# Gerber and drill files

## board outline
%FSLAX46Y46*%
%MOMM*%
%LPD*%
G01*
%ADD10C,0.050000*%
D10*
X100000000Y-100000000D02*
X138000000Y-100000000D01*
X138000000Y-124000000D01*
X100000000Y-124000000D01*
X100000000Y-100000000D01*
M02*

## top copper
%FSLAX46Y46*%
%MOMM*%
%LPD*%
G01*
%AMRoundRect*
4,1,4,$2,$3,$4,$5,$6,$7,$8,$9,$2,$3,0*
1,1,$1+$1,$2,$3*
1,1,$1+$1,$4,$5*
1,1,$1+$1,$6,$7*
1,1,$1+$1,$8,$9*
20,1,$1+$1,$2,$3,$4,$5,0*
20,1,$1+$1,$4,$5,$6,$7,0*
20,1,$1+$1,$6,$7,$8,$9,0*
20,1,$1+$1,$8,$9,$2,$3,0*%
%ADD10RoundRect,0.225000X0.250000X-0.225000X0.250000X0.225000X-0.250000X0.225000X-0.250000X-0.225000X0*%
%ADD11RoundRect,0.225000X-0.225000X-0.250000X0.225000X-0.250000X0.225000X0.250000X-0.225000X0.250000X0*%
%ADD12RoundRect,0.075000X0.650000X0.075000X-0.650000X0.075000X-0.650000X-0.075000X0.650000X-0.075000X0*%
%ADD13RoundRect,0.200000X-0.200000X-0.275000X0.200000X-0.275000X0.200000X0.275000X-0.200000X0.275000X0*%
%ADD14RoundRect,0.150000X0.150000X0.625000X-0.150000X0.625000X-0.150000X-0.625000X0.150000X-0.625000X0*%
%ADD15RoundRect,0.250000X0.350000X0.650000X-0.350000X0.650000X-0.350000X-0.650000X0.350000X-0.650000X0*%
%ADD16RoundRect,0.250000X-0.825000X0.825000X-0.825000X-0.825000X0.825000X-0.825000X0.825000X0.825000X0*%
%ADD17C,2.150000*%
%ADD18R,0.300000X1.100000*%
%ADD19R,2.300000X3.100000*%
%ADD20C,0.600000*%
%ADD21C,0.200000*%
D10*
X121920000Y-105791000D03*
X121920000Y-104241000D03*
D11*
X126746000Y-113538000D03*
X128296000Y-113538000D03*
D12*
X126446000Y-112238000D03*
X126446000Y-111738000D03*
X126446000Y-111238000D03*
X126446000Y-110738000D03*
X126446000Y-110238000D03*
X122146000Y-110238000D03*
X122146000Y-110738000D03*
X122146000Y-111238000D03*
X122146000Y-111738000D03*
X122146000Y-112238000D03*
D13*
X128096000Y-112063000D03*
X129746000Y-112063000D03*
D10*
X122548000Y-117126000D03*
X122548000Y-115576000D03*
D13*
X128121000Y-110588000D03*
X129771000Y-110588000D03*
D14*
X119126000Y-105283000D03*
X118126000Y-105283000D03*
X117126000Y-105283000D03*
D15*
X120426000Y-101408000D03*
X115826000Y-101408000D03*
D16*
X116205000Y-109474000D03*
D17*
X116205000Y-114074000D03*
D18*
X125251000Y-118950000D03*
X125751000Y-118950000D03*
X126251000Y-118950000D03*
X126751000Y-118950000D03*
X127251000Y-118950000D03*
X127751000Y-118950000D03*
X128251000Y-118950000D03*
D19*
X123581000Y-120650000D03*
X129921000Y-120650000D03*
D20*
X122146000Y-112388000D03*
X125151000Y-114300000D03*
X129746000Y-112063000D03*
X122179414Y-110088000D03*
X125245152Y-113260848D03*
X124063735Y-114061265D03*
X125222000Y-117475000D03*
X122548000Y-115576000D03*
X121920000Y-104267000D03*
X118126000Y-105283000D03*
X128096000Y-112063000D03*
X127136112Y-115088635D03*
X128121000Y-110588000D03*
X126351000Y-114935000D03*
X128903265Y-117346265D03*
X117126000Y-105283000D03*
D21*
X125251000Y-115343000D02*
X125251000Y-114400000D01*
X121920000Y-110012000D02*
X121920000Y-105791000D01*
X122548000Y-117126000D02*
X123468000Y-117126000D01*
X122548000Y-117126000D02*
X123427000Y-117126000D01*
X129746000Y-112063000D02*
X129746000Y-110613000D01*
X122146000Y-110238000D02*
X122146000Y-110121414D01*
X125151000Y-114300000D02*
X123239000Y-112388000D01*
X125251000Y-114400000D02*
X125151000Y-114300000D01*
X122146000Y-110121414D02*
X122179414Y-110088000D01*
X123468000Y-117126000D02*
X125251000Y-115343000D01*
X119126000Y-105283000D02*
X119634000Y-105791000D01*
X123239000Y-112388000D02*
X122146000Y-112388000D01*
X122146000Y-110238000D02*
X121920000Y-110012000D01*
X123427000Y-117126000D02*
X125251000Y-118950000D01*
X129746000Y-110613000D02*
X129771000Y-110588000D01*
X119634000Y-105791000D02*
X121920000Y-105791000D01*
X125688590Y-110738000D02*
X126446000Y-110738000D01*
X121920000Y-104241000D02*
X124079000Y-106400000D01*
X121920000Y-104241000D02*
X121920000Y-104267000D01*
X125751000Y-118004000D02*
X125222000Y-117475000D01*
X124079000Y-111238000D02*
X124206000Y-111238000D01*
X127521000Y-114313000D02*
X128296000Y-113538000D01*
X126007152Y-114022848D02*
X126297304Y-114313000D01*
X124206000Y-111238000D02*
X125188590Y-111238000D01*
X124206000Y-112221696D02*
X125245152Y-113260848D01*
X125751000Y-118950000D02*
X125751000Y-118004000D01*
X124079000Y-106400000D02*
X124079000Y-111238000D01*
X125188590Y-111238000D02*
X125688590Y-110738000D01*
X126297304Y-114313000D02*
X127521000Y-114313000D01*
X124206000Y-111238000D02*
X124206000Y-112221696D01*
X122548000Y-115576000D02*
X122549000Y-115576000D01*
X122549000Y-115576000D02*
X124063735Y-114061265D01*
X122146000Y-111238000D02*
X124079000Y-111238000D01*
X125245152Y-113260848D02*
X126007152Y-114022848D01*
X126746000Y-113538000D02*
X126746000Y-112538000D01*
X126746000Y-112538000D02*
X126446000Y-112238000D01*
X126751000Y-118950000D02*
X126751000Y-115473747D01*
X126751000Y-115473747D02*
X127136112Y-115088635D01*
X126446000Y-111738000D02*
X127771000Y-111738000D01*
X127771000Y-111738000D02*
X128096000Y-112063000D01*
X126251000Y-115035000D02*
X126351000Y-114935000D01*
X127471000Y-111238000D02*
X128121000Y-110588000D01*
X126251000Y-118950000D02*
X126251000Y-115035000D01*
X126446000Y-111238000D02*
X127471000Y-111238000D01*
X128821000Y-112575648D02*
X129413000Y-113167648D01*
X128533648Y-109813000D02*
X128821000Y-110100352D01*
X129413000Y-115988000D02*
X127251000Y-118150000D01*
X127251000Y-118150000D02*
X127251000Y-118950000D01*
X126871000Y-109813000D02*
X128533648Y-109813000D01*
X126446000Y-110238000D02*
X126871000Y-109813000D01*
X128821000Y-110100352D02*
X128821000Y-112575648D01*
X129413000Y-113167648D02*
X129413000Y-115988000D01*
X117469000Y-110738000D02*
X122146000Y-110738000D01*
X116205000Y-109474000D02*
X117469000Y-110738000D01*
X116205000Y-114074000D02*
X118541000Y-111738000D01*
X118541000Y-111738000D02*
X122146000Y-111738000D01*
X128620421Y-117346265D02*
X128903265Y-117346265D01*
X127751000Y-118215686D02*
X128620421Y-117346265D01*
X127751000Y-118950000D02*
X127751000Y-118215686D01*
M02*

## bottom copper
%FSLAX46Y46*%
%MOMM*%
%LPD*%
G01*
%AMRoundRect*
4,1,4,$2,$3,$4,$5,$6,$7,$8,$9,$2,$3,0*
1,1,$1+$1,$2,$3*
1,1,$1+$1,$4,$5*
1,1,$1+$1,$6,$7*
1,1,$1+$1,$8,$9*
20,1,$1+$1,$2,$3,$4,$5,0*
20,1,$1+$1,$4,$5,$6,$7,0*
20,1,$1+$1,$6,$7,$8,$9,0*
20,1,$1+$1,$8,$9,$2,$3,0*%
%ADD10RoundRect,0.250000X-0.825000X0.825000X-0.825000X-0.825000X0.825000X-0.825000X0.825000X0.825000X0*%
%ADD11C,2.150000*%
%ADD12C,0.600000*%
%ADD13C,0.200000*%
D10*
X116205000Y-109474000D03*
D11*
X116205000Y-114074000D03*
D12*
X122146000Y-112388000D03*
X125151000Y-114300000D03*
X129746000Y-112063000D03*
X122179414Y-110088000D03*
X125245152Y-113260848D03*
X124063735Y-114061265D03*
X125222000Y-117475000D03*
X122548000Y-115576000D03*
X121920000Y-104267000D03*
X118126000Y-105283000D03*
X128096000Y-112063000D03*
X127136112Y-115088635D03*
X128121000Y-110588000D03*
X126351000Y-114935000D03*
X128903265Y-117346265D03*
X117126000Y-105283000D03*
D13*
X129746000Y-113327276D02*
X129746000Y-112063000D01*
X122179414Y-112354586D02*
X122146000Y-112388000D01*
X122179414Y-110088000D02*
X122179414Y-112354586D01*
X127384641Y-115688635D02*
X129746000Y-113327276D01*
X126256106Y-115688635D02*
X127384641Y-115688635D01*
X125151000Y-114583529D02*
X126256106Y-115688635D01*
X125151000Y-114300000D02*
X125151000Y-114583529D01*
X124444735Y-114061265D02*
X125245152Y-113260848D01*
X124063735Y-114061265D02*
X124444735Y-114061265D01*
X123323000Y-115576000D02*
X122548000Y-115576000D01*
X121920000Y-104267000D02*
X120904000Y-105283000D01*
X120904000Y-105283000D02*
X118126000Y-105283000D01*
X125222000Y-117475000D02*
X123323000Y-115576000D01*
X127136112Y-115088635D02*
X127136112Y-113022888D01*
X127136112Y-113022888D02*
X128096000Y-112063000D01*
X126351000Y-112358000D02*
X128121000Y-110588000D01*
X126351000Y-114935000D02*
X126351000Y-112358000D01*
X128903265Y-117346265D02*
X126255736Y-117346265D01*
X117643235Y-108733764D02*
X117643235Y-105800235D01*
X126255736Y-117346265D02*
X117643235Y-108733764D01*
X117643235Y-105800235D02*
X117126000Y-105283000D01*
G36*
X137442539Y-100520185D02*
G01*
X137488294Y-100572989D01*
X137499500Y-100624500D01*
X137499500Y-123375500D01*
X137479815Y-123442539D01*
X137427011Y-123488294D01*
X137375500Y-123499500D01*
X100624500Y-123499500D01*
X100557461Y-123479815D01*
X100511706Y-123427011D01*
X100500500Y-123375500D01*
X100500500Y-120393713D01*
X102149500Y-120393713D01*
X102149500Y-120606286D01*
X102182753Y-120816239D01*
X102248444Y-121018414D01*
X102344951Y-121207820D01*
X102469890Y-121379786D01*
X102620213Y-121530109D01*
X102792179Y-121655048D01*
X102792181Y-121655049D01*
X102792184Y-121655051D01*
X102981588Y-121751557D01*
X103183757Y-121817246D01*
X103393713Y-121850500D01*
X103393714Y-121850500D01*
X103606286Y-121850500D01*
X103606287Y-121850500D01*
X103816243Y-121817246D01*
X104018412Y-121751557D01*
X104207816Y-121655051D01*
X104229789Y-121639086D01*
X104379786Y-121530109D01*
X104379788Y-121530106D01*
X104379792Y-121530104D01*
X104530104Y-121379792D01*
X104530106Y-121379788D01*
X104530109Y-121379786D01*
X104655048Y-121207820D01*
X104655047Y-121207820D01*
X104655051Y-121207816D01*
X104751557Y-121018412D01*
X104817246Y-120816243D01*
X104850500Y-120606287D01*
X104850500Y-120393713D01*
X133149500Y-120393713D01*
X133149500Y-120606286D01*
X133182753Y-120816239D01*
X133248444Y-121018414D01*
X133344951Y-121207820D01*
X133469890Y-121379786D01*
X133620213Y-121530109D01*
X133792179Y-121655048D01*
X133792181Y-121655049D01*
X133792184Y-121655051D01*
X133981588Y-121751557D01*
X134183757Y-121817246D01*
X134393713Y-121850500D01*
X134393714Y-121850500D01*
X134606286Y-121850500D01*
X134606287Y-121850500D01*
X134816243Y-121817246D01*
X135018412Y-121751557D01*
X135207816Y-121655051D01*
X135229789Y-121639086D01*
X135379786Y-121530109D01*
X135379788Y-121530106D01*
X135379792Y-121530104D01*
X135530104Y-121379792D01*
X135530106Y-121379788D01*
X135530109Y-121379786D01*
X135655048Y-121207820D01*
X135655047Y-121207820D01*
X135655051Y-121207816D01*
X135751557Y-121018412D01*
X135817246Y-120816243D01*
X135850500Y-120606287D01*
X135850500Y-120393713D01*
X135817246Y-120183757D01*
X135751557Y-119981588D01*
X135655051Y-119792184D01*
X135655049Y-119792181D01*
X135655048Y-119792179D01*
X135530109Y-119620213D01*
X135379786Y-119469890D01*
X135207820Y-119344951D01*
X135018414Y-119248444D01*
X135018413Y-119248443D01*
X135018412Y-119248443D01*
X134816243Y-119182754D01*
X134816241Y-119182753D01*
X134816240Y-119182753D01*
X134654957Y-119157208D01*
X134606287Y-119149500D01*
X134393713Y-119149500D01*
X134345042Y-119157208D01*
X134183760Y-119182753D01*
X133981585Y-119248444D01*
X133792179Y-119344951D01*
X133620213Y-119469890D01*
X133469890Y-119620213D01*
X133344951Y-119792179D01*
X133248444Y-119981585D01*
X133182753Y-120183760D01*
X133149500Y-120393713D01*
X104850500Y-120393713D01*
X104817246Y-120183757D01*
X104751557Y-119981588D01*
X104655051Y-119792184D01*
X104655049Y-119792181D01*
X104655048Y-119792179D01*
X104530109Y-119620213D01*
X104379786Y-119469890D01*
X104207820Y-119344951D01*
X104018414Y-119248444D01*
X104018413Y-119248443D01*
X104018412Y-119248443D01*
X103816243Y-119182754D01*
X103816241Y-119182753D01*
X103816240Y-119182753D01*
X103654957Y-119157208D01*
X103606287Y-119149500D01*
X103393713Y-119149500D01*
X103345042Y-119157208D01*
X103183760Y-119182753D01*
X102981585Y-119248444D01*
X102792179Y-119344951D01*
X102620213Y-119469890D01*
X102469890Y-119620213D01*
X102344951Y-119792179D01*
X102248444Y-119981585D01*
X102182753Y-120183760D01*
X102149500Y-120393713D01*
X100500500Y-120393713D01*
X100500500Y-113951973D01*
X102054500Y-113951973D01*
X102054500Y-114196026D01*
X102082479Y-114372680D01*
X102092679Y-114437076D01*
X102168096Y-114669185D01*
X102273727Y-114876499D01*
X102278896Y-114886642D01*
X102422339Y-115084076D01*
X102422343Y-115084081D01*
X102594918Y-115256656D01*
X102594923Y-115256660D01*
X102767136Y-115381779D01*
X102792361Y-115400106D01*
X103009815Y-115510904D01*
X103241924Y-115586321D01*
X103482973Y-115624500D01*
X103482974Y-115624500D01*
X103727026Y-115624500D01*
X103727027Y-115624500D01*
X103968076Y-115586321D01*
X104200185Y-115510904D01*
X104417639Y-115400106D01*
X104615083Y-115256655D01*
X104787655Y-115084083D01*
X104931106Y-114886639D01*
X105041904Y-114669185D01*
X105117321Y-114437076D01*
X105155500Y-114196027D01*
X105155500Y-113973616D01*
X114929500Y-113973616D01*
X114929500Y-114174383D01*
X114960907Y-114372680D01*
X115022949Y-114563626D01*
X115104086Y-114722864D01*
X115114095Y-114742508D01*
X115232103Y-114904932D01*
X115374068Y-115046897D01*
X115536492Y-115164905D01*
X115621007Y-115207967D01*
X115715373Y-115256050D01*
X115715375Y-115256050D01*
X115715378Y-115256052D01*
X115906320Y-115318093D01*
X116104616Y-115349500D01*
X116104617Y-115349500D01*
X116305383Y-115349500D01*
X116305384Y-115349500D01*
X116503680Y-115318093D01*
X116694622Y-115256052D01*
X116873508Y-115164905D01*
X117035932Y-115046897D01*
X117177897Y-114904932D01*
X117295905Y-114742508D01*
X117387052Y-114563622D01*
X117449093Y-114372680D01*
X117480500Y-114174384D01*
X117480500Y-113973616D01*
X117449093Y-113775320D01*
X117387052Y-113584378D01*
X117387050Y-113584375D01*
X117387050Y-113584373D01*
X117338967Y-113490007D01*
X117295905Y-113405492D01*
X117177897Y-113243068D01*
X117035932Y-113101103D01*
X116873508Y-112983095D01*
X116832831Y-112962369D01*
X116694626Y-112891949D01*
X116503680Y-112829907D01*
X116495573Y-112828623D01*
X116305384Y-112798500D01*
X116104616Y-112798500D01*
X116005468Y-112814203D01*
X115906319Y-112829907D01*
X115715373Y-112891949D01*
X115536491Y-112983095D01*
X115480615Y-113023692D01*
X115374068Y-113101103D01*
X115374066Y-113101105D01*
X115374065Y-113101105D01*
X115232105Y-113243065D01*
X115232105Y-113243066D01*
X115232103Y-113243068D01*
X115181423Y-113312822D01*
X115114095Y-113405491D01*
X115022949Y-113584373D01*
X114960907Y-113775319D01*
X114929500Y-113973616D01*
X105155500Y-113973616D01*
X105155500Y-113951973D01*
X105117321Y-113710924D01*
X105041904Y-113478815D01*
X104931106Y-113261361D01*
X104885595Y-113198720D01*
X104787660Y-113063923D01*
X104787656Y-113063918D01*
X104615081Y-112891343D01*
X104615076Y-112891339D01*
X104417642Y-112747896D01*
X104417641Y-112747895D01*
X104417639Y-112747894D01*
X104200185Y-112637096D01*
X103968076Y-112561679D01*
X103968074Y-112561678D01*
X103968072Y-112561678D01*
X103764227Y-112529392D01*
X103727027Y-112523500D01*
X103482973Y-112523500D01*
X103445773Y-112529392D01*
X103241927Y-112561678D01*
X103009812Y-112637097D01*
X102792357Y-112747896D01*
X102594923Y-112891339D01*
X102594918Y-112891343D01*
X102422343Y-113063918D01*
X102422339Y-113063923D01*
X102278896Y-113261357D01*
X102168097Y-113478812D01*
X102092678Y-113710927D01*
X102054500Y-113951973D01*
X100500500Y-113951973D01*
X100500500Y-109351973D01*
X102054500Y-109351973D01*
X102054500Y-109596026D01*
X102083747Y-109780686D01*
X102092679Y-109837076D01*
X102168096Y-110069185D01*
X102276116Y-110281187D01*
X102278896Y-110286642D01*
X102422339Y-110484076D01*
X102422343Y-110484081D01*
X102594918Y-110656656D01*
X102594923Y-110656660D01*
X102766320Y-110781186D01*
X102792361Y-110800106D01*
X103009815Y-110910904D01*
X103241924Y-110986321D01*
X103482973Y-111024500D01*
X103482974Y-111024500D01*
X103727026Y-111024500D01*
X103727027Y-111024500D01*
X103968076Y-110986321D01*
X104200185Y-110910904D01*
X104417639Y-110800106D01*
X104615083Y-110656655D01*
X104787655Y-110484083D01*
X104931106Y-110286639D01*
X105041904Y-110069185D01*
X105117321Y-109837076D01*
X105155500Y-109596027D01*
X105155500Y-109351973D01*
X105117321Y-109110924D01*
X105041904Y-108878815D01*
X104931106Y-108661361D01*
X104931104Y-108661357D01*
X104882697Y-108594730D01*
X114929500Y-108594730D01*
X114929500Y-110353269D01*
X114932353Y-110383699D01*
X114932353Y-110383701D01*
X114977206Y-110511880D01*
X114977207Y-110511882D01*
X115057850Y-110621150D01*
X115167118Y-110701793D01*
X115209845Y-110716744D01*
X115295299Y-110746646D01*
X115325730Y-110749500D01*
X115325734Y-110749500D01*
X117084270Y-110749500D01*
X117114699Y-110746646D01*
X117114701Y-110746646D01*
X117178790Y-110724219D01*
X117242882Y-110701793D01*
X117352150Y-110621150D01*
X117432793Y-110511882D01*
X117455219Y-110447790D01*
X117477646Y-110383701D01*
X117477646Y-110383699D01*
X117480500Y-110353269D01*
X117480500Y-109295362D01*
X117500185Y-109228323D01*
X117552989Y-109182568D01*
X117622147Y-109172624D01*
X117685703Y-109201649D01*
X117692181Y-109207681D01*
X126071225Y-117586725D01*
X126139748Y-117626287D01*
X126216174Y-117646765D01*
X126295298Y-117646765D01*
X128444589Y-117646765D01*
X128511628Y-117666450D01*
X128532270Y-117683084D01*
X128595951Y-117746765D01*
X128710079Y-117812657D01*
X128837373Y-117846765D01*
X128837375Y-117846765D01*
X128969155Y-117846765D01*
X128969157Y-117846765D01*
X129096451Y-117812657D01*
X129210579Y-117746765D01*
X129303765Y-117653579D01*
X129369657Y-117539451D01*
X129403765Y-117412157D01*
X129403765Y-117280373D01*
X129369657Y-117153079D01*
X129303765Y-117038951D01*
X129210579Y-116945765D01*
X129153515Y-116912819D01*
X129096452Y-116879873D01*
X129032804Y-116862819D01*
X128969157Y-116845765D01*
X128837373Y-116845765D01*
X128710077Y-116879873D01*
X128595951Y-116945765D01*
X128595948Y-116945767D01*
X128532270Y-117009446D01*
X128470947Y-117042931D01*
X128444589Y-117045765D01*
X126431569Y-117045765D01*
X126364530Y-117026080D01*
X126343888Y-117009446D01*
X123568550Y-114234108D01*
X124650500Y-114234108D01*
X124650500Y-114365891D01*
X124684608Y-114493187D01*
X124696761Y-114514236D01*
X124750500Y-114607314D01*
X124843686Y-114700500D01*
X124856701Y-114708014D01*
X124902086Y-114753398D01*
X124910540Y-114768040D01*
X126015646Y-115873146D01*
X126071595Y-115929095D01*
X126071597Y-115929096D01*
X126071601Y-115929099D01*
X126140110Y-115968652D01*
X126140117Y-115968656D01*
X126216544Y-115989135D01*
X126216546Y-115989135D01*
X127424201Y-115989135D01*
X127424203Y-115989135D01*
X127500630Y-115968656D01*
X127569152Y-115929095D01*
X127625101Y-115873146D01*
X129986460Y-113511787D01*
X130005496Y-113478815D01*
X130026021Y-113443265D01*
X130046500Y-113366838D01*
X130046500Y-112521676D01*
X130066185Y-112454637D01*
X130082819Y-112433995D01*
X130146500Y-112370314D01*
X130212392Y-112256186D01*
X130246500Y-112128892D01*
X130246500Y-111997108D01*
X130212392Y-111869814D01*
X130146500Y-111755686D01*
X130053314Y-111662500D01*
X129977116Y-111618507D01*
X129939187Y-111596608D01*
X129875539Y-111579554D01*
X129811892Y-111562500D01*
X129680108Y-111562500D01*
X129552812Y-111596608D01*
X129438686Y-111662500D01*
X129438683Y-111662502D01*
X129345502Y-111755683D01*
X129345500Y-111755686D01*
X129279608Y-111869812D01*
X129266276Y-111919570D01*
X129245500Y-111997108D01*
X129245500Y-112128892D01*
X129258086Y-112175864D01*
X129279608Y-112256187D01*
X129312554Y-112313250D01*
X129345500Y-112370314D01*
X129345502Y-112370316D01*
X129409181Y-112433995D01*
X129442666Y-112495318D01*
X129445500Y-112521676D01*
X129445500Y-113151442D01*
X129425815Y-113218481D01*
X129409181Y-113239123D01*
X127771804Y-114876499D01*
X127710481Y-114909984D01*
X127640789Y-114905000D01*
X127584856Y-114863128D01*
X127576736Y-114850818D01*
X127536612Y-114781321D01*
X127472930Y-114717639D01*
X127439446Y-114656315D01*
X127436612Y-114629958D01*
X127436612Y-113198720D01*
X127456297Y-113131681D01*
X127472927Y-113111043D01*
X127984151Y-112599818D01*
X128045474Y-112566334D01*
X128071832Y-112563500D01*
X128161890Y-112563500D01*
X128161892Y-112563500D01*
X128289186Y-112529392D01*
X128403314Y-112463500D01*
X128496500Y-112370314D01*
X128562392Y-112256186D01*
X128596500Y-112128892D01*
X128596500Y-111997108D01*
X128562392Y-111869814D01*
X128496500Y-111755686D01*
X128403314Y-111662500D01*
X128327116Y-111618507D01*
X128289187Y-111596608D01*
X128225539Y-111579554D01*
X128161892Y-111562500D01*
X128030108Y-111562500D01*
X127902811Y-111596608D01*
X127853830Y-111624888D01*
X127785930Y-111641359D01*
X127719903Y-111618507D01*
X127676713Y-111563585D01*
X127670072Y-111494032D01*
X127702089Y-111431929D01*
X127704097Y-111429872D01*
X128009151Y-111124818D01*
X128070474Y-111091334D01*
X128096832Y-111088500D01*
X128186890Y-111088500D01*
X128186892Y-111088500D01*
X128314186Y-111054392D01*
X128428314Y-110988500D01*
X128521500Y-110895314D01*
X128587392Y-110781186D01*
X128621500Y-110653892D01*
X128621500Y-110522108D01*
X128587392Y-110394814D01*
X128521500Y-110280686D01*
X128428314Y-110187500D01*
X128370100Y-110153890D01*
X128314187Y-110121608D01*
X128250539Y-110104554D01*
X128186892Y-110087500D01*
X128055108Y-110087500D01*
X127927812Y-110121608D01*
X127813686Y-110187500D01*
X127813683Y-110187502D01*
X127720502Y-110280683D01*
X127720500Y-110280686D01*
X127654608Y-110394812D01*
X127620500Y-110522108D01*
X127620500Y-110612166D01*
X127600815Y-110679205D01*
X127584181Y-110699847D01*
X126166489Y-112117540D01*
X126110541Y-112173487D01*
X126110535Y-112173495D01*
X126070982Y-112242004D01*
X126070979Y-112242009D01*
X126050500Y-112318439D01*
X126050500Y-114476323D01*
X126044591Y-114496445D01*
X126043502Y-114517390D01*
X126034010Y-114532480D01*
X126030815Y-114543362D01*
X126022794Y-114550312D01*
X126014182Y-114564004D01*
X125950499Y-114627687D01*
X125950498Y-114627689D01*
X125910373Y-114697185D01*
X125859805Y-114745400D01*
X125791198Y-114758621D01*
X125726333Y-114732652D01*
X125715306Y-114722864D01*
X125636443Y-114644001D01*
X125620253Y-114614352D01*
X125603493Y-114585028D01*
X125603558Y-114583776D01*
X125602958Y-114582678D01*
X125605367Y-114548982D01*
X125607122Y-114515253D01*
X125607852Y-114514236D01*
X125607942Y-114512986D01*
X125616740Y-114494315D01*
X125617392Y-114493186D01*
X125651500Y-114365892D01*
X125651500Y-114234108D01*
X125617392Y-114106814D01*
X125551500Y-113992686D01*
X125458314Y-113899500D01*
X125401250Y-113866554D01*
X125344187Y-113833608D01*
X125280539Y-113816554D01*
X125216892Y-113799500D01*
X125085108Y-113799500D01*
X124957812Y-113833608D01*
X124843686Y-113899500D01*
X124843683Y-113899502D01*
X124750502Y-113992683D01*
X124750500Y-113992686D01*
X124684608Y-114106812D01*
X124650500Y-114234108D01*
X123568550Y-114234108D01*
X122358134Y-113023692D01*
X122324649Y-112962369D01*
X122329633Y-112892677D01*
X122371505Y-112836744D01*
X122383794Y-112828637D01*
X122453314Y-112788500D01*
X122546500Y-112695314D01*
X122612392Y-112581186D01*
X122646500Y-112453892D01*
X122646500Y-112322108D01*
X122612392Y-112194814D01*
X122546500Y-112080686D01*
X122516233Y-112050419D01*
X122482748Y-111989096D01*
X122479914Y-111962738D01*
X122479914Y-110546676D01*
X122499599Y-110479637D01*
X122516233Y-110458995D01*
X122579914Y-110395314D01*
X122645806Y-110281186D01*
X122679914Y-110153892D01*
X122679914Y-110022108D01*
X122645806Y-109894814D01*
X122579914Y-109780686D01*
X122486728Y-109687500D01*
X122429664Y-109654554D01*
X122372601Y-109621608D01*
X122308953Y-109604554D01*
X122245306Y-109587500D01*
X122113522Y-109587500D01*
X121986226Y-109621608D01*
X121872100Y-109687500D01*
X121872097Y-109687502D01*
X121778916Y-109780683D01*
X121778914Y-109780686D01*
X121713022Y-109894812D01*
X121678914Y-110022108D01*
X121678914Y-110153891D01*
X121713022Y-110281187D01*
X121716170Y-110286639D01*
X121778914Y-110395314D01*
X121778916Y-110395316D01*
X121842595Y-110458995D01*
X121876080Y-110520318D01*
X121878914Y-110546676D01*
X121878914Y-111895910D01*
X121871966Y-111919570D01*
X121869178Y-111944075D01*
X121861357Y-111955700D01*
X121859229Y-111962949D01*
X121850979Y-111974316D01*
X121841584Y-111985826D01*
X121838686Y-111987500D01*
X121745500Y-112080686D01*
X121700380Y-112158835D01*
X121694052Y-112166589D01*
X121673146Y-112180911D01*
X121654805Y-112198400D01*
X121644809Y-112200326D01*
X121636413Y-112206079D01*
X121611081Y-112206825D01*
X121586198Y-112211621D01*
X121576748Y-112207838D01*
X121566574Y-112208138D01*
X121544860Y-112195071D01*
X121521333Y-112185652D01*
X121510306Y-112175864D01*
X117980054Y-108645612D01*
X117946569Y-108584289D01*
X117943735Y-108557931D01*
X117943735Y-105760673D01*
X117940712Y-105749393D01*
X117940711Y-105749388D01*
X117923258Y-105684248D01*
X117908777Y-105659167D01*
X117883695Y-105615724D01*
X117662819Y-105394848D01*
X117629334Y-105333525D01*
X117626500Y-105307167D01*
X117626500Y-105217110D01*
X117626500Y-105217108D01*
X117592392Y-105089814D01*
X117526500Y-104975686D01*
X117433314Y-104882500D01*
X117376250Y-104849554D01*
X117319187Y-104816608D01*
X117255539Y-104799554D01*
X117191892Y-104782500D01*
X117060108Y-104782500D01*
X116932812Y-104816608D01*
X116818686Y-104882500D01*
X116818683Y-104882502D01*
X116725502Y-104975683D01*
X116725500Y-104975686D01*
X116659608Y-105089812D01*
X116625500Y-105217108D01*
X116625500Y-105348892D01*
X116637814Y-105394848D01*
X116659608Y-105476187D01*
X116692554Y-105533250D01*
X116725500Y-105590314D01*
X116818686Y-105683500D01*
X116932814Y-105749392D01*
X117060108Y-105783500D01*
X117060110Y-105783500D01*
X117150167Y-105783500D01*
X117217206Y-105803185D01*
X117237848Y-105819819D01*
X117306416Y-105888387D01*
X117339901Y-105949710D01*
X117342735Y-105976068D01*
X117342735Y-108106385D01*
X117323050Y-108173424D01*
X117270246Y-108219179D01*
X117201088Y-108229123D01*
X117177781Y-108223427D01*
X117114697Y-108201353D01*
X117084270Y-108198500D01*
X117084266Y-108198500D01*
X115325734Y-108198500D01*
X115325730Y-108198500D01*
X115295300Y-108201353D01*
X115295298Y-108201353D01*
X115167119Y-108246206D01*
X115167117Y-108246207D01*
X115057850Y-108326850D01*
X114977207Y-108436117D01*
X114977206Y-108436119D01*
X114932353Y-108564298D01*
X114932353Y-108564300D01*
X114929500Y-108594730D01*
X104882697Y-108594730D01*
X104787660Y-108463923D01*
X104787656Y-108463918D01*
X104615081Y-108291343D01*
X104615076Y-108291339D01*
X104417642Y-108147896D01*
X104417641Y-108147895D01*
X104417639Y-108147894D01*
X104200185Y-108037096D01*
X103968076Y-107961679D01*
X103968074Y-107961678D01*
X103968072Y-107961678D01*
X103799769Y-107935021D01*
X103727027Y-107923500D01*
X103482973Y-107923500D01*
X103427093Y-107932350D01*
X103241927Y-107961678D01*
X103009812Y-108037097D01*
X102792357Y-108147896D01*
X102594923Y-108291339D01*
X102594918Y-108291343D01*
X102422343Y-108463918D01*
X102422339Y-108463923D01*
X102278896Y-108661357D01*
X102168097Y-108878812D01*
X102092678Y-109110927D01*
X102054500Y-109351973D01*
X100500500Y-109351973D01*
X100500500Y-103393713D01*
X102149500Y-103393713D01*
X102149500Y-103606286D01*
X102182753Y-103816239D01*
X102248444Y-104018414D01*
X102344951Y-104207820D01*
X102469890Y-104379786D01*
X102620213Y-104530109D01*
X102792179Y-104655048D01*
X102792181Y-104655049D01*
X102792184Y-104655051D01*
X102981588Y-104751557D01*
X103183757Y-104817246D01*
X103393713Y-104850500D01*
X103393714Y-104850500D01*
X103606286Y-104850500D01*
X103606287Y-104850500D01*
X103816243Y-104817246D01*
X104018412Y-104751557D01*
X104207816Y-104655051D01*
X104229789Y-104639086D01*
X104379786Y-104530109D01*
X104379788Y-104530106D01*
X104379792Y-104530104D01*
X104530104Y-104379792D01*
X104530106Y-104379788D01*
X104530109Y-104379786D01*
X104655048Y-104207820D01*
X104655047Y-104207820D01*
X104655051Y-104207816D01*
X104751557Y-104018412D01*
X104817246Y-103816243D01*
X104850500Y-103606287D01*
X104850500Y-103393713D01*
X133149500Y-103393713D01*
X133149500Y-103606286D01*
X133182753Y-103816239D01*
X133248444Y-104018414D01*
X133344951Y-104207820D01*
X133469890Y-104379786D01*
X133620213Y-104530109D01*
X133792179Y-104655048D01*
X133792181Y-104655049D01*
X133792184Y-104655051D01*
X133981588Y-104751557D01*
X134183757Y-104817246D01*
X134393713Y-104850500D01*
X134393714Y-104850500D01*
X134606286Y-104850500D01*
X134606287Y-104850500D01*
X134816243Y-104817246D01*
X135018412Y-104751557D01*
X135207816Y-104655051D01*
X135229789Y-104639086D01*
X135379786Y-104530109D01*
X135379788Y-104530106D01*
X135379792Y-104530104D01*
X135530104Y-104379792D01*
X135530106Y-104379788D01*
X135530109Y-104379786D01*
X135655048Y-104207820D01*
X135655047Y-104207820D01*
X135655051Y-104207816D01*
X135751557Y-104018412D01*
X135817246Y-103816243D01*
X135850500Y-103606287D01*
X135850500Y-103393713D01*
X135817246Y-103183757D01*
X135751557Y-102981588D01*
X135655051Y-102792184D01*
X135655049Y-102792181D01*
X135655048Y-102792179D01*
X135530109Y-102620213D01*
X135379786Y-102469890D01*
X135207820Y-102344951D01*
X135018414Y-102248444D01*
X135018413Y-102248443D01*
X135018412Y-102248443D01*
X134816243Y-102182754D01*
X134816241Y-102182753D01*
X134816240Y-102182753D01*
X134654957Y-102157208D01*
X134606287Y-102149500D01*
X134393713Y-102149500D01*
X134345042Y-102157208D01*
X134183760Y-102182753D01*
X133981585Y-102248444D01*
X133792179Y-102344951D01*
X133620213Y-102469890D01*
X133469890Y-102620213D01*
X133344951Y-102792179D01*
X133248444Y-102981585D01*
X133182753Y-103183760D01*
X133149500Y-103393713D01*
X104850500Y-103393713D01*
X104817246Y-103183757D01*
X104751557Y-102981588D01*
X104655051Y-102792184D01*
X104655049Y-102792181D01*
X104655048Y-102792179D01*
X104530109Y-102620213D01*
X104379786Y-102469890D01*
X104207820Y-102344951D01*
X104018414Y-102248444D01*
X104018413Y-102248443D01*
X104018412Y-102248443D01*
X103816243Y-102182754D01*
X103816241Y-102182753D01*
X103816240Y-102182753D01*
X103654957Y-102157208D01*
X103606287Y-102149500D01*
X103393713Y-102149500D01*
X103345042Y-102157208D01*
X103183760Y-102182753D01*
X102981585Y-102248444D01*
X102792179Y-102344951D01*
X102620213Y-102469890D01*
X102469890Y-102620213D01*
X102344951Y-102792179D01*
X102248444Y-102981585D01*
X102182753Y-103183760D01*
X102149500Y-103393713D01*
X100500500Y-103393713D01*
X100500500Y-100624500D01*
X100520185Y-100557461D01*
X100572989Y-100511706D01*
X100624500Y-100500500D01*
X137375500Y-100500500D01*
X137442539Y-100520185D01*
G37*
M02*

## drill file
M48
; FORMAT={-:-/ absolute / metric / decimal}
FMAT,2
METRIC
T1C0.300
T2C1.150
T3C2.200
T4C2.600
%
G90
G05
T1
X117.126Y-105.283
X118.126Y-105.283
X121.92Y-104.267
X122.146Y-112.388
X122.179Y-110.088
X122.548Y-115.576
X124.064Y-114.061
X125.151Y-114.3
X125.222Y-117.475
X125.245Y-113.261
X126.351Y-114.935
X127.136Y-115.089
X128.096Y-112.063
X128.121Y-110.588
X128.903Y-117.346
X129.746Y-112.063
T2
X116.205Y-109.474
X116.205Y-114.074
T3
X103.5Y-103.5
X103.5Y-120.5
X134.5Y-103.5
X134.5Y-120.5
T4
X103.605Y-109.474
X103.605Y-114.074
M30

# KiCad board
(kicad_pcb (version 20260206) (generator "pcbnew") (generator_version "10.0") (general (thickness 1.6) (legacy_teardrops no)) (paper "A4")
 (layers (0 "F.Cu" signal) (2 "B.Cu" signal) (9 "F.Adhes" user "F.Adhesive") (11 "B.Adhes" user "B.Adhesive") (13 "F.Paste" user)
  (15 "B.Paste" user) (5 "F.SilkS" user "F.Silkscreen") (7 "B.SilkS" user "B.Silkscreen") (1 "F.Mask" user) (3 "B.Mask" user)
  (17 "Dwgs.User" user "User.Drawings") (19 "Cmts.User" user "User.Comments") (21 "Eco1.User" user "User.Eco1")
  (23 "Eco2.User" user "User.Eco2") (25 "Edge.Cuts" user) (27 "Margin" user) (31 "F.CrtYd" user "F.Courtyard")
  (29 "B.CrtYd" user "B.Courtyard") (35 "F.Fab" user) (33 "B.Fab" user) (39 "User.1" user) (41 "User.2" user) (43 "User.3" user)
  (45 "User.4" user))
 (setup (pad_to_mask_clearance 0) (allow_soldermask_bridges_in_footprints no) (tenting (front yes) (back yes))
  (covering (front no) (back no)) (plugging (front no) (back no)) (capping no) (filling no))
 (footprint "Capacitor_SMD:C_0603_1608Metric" (layer "F.Cu") (at 121.92 105.016 90)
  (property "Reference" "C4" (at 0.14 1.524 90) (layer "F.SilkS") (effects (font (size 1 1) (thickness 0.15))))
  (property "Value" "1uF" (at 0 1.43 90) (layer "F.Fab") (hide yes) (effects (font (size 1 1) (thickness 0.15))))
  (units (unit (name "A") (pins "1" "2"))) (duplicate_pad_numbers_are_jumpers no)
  (pad "1" smd roundrect (at -0.775 0 90) (size 0.9 0.95) (layers "F.Cu" "F.Mask" "F.Paste") (roundrect_rratio 0.25) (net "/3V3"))
  (pad "2" smd roundrect (at 0.775 0 90) (size 0.9 0.95) (layers "F.Cu" "F.Mask" "F.Paste") (roundrect_rratio 0.25) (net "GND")))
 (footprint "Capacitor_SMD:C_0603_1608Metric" (layer "F.Cu") (at 127.521 113.538)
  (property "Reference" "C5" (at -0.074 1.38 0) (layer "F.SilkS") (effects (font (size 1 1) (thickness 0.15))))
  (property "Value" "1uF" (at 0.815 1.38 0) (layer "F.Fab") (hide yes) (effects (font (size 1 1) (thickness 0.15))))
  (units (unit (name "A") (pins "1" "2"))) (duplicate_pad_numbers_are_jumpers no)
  (pad "1" smd roundrect (at -0.775 0) (size 0.9 0.95) (layers "F.Cu" "F.Mask" "F.Paste") (roundrect_rratio 0.25) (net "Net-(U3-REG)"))
  (pad "2" smd roundrect (at 0.775 0) (size 0.9 0.95) (layers "F.Cu" "F.Mask" "F.Paste") (roundrect_rratio 0.25) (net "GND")))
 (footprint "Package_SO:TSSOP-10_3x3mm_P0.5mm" (layer "F.Cu") (at 124.296 111.238 180)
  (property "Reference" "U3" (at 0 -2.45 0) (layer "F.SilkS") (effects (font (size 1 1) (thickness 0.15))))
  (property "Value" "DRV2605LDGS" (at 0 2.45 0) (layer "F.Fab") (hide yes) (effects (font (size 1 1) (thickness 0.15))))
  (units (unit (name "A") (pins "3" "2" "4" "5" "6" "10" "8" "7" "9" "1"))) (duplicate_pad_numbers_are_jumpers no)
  (pad "1" smd roundrect (at -2.15 -1 180) (size 1.45 0.3) (layers "F.Cu" "F.Mask" "F.Paste") (roundrect_rratio 0.25) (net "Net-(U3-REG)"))
  (pad "2" smd roundrect (at -2.15 -0.5 180) (size 1.45 0.3) (layers "F.Cu" "F.Mask" "F.Paste") (roundrect_rratio 0.25) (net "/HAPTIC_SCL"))
  (pad "3" smd roundrect (at -2.15 0 180) (size 1.45 0.3) (layers "F.Cu" "F.Mask" "F.Paste") (roundrect_rratio 0.25) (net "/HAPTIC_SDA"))
  (pad "4" smd roundrect (at -2.15 0.5 180) (size 1.45 0.3) (layers "F.Cu" "F.Mask" "F.Paste") (roundrect_rratio 0.25) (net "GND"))
  (pad "5" smd roundrect (at -2.15 1 180) (size 1.45 0.3) (layers "F.Cu" "F.Mask" "F.Paste") (roundrect_rratio 0.25) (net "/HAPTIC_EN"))
  (pad "6" smd roundrect (at 2.15 1 180) (size 1.45 0.3) (layers "F.Cu" "F.Mask" "F.Paste") (roundrect_rratio 0.25) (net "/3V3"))
  (pad "7" smd roundrect (at 2.15 0.5 180) (size 1.45 0.3) (layers "F.Cu" "F.Mask" "F.Paste") (roundrect_rratio 0.25) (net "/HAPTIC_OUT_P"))
  (pad "8" smd roundrect (at 2.15 0 180) (size 1.45 0.3) (layers "F.Cu" "F.Mask" "F.Paste") (roundrect_rratio 0.25) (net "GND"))
  (pad "9" smd roundrect (at 2.15 -0.5 180) (size 1.45 0.3) (layers "F.Cu" "F.Mask" "F.Paste") (roundrect_rratio 0.25) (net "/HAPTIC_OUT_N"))
  (pad "10" smd roundrect (at 2.15 -1 180) (size 1.45 0.3) (layers "F.Cu" "F.Mask" "F.Paste") (roundrect_rratio 0.25) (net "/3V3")))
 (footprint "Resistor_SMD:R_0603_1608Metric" (layer "F.Cu") (at 128.921 112.063)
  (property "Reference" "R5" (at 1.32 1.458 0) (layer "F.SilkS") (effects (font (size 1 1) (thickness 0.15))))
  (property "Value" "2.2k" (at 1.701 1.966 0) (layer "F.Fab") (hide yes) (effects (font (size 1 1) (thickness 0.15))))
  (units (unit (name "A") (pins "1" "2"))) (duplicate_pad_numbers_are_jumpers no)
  (pad "1" smd roundrect (at -0.825 0) (size 0.8 0.95) (layers "F.Cu" "F.Mask" "F.Paste") (roundrect_rratio 0.25) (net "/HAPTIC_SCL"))
  (pad "2" smd roundrect (at 0.825 0) (size 0.8 0.95) (layers "F.Cu" "F.Mask" "F.Paste") (roundrect_rratio 0.25) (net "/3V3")))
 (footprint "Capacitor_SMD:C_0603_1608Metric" (layer "F.Cu") (at 122.548 116.351 90)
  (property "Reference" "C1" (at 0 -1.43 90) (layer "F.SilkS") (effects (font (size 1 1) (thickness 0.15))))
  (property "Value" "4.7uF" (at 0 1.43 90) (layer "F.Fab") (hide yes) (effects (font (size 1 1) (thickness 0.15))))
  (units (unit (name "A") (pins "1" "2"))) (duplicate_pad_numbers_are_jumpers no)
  (pad "1" smd roundrect (at -0.775 0 90) (size 0.9 0.95) (layers "F.Cu" "F.Mask" "F.Paste") (roundrect_rratio 0.25) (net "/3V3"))
  (pad "2" smd roundrect (at 0.775 0 90) (size 0.9 0.95) (layers "F.Cu" "F.Mask" "F.Paste") (roundrect_rratio 0.25) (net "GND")))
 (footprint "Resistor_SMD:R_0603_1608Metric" (layer "F.Cu") (at 128.946 110.588)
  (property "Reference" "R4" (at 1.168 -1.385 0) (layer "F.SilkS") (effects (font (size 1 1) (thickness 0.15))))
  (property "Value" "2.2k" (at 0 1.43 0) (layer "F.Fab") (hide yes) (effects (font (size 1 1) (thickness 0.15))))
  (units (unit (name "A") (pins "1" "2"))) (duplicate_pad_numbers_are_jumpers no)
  (pad "1" smd roundrect (at -0.825 0) (size 0.8 0.95) (layers "F.Cu" "F.Mask" "F.Paste") (roundrect_rratio 0.25) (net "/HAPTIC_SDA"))
  (pad "2" smd roundrect (at 0.825 0) (size 0.8 0.95) (layers "F.Cu" "F.Mask" "F.Paste") (roundrect_rratio 0.25) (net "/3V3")))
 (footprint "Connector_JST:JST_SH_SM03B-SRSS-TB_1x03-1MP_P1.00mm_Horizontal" (layer "F.Cu") (at 118.126 103.283 180)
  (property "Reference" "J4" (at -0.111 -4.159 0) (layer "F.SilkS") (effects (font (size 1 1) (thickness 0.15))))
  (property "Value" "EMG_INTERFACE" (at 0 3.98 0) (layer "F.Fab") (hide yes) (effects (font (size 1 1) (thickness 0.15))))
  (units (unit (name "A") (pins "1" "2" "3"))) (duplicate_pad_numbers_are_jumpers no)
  (pad "1" smd roundrect (at -1 -2 180) (size 0.6 1.55) (layers "F.Cu" "F.Mask" "F.Paste") (roundrect_rratio 0.25) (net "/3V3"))
  (pad "2" smd roundrect (at 0 -2 180) (size 0.6 1.55) (layers "F.Cu" "F.Mask" "F.Paste") (roundrect_rratio 0.25) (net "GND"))
  (pad "3" smd roundrect (at 1 -2 180) (size 0.6 1.55) (layers "F.Cu" "F.Mask" "F.Paste") (roundrect_rratio 0.25) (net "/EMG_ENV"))
  (pad "MP" smd roundrect (at -2.3 1.875 180) (size 1.2 1.8) (layers "F.Cu" "F.Mask" "F.Paste") (roundrect_rratio 0.208333))
  (pad "MP" smd roundrect (at 2.3 1.875 180) (size 1.2 1.8) (layers "F.Cu" "F.Mask" "F.Paste") (roundrect_rratio 0.208333)))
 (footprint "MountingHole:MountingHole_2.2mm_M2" (layer "F.Cu") (at 103.5 103.5)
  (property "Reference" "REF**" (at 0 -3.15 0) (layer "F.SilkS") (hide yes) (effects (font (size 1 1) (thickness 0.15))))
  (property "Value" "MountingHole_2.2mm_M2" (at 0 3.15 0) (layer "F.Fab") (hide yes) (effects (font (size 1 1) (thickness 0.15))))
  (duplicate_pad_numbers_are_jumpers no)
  (pad "" np_thru_hole circle (at 0 0) (size 2.2 2.2) (drill 2.2) (layers "*.Cu" "*.Mask")))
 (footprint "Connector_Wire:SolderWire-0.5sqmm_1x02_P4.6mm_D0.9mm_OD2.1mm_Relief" (layer "F.Cu") (at 116.205 109.474 -90)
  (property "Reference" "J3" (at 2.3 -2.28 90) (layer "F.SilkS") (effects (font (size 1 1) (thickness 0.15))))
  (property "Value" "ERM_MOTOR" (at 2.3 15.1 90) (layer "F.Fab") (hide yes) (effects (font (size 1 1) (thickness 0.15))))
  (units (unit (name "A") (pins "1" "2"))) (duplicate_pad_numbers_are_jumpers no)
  (pad "" np_thru_hole circle (at 0 12.6 270) (size 2.6 2.6) (drill 2.6) (layers "*.Cu" "*.Mask"))
  (pad "" np_thru_hole circle (at 4.6 12.6 270) (size 2.6 2.6) (drill 2.6) (layers "*.Cu" "*.Mask"))
  (pad "1" thru_hole roundrect (at 0 0 270) (size 2.15 2.15) (drill 1.15) (layers "*.Cu" "*.Mask") (remove_unused_layers no)
   (roundrect_rratio 0.116279) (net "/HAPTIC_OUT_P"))
  (pad "2" thru_hole circle (at 4.6 0 270) (size 2.15 2.15) (drill 1.15) (layers "*.Cu" "*.Mask") (remove_unused_layers no)
   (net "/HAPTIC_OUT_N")))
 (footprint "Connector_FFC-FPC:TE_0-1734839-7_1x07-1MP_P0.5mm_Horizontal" (layer "F.Cu") (at 126.751 120.3)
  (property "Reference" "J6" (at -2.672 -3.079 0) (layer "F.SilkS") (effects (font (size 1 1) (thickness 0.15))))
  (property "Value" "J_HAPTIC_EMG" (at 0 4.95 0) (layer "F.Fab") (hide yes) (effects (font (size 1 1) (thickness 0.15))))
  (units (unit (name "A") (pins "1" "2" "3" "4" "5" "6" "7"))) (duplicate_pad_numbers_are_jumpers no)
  (pad "1" smd rect (at -1.5 -1.35) (size 0.3 1.1) (layers "F.Cu" "F.Mask" "F.Paste") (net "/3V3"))
  (pad "2" smd rect (at -1 -1.35) (size 0.3 1.1) (layers "F.Cu" "F.Mask" "F.Paste") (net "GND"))
  (pad "3" smd rect (at -0.5 -1.35) (size 0.3 1.1) (layers "F.Cu" "F.Mask" "F.Paste") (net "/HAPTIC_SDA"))
  (pad "4" smd rect (at 0 -1.35) (size 0.3 1.1) (layers "F.Cu" "F.Mask" "F.Paste") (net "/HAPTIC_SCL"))
  (pad "5" smd rect (at 0.5 -1.35) (size 0.3 1.1) (layers "F.Cu" "F.Mask" "F.Paste") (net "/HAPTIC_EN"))
  (pad "6" smd rect (at 1 -1.35) (size 0.3 1.1) (layers "F.Cu" "F.Mask" "F.Paste") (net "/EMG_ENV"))
  (pad "7" smd rect (at 1.5 -1.35) (size 0.3 1.1) (layers "F.Cu" "F.Mask" "F.Paste") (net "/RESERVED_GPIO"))
  (pad "MP" smd rect (at -3.17 0.35) (size 2.3 3.1) (layers "F.Cu" "F.Mask" "F.Paste"))
  (pad "MP" smd rect (at 3.17 0.35) (size 2.3 3.1) (layers "F.Cu" "F.Mask" "F.Paste")))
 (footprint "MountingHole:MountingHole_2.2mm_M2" (layer "F.Cu") (at 134.5 120.5)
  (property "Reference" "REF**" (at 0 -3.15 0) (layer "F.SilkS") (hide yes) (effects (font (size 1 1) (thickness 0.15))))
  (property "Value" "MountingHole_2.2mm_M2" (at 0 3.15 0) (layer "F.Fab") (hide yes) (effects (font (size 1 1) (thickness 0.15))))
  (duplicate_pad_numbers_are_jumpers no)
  (pad "" np_thru_hole circle (at 0 0) (size 2.2 2.2) (drill 2.2) (layers "*.Cu" "*.Mask")))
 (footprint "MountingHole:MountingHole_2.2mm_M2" (layer "F.Cu") (at 134.5 103.5)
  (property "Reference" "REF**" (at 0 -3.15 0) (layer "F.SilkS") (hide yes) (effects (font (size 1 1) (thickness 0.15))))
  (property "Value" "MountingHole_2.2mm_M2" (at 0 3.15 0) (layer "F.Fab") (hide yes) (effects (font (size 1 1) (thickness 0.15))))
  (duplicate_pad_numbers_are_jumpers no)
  (pad "" np_thru_hole circle (at 0 0) (size 2.2 2.2) (drill 2.2) (layers "*.Cu" "*.Mask")))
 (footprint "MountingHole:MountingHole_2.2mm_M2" (layer "F.Cu") (at 103.5 120.5)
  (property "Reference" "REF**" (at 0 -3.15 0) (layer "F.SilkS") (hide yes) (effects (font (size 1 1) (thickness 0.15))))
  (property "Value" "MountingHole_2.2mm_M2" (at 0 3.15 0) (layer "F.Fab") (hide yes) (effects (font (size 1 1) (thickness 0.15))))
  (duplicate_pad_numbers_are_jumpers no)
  (pad "" np_thru_hole circle (at 0 0) (size 2.2 2.2) (drill 2.2) (layers "*.Cu" "*.Mask")))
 (gr_rect (start 100 100) (end 138 124) (stroke (width 0.05) (type solid)) (fill no) (layer "Edge.Cuts"))
 (segment (start 125.251 115.343) (end 125.251 114.4) (width 0.2) (layer "F.Cu") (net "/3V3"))
 (segment (start 121.92 110.012) (end 121.92 105.791) (width 0.2) (layer "F.Cu") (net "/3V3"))
 (segment (start 122.548 117.126) (end 123.468 117.126) (width 0.2) (layer "F.Cu") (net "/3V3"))
 (segment (start 122.548 117.126) (end 123.427 117.126) (width 0.2) (layer "F.Cu") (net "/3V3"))
 (segment (start 129.746 112.063) (end 129.746 110.613) (width 0.2) (layer "F.Cu") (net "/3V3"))
 (segment (start 122.146 110.238) (end 122.146 110.121414) (width 0.2) (layer "F.Cu") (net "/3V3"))
 (segment (start 125.151 114.3) (end 123.239 112.388) (width 0.2) (layer "F.Cu") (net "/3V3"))
 (segment (start 125.251 114.4) (end 125.151 114.3) (width 0.2) (layer "F.Cu") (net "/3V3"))
 (segment (start 122.146 110.121414) (end 122.179414 110.088) (width 0.2) (layer "F.Cu") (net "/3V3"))
 (segment (start 123.468 117.126) (end 125.251 115.343) (width 0.2) (layer "F.Cu") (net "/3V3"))
 (segment (start 119.126 105.283) (end 119.634 105.791) (width 0.2) (layer "F.Cu") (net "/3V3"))
 (segment (start 123.239 112.388) (end 122.146 112.388) (width 0.2) (layer "F.Cu") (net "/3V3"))
 (segment (start 122.146 110.238) (end 121.92 110.012) (width 0.2) (layer "F.Cu") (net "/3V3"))
 (segment (start 123.427 117.126) (end 125.251 118.95) (width 0.2) (layer "F.Cu") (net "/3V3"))
 (segment (start 129.746 110.613) (end 129.771 110.588) (width 0.2) (layer "F.Cu") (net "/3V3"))
 (segment (start 119.634 105.791) (end 121.92 105.791) (width 0.2) (layer "F.Cu") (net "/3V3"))
 (via (at 122.146 112.388) (size 0.6) (drill 0.3) (layers "F.Cu" "B.Cu") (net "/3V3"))
 (via (at 125.151 114.3) (size 0.6) (drill 0.3) (layers "F.Cu" "B.Cu") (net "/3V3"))
 (via (at 129.746 112.063) (size 0.6) (drill 0.3) (layers "F.Cu" "B.Cu") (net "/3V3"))
 (via (at 122.179414 110.088) (size 0.6) (drill 0.3) (layers "F.Cu" "B.Cu") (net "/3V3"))
 (segment (start 129.746 113.327276) (end 129.746 112.063) (width 0.2) (layer "B.Cu") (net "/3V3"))
 (segment (start 122.179414 112.354586) (end 122.146 112.388) (width 0.2) (layer "B.Cu") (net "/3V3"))
 (segment (start 122.179414 110.088) (end 122.179414 112.354586) (width 0.2) (layer "B.Cu") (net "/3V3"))
 (segment (start 127.384641 115.688635) (end 129.746 113.327276) (width 0.2) (layer "B.Cu") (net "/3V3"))
 (segment (start 126.256106 115.688635) (end 127.384641 115.688635) (width 0.2) (layer "B.Cu") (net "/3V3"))
 (segment (start 125.151 114.583529) (end 126.256106 115.688635) (width 0.2) (layer "B.Cu") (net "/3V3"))
 (segment (start 125.151 114.3) (end 125.151 114.583529) (width 0.2) (layer "B.Cu") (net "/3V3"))
 (segment (start 125.68859 110.738) (end 126.446 110.738) (width 0.2) (layer "F.Cu") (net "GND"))
 (segment (start 121.92 104.241) (end 124.079 106.4) (width 0.2) (layer "F.Cu") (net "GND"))
 (segment (start 121.92 104.241) (end 121.92 104.267) (width 0.2) (layer "F.Cu") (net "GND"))
 (segment (start 125.751 118.004) (end 125.222 117.475) (width 0.2) (layer "F.Cu") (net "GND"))
 (segment (start 124.079 111.238) (end 124.206 111.238) (width 0.2) (layer "F.Cu") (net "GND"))
 (segment (start 127.521 114.313) (end 128.296 113.538) (width 0.2) (layer "F.Cu") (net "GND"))
 (segment (start 126.007152 114.022848) (end 126.297304 114.313) (width 0.2) (layer "F.Cu") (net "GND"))
 (segment (start 124.206 111.238) (end 125.18859 111.238) (width 0.2) (layer "F.Cu") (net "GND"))
 (segment (start 124.206 112.221696) (end 125.245152 113.260848) (width 0.2) (layer "F.Cu") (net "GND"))
 (segment (start 125.751 118.95) (end 125.751 118.004) (width 0.2) (layer "F.Cu") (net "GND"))
 (segment (start 124.079 106.4) (end 124.079 111.238) (width 0.2) (layer "F.Cu") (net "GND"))
 (segment (start 125.18859 111.238) (end 125.68859 110.738) (width 0.2) (layer "F.Cu") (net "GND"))
 (segment (start 126.297304 114.313) (end 127.521 114.313) (width 0.2) (layer "F.Cu") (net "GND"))
 (segment (start 124.206 111.238) (end 124.206 112.221696) (width 0.2) (layer "F.Cu") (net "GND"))
 (segment (start 122.548 115.576) (end 122.549 115.576) (width 0.2) (layer "F.Cu") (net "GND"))
 (segment (start 122.549 115.576) (end 124.063735 114.061265) (width 0.2) (layer "F.Cu") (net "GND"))
 (segment (start 122.146 111.238) (end 124.079 111.238) (width 0.2) (layer "F.Cu") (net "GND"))
 (segment (start 125.245152 113.260848) (end 126.007152 114.022848) (width 0.2) (layer "F.Cu") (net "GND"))
 (via (at 125.245152 113.260848) (size 0.6) (drill 0.3) (layers "F.Cu" "B.Cu") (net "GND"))
 (via (at 124.063735 114.061265) (size 0.6) (drill 0.3) (layers "F.Cu" "B.Cu") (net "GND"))
 (via (at 125.222 117.475) (size 0.6) (drill 0.3) (layers "F.Cu" "B.Cu") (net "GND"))
 (via (at 122.548 115.576) (size 0.6) (drill 0.3) (layers "F.Cu" "B.Cu") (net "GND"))
 (via (at 121.92 104.267) (size 0.6) (drill 0.3) (layers "F.Cu" "B.Cu") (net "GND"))
 (via (at 118.126 105.283) (size 0.6) (drill 0.3) (layers "F.Cu" "B.Cu") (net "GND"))
 (segment (start 124.444735 114.061265) (end 125.245152 113.260848) (width 0.2) (layer "B.Cu") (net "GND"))
 (segment (start 124.063735 114.061265) (end 124.444735 114.061265) (width 0.2) (layer "B.Cu") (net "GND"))
 (segment (start 123.323 115.576) (end 122.548 115.576) (width 0.2) (layer "B.Cu") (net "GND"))
 (segment (start 121.92 104.267) (end 120.904 105.283) (width 0.2) (layer "B.Cu") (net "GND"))
 (segment (start 120.904 105.283) (end 118.126 105.283) (width 0.2) (layer "B.Cu") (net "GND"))
 (segment (start 125.222 117.475) (end 123.323 115.576) (width 0.2) (layer "B.Cu") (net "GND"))
 (segment (start 126.746 113.538) (end 126.746 112.538) (width 0.2) (layer "F.Cu") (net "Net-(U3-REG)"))
 (segment (start 126.746 112.538) (end 126.446 112.238) (width 0.2) (layer "F.Cu") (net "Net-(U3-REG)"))
 (segment (start 126.751 118.95) (end 126.751 115.473747) (width 0.2) (layer "F.Cu") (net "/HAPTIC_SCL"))
 (segment (start 126.751 115.473747) (end 127.136112 115.088635) (width 0.2) (layer "F.Cu") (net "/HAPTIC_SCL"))
 (segment (start 126.446 111.738) (end 127.771 111.738) (width 0.2) (layer "F.Cu") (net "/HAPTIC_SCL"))
 (segment (start 127.771 111.738) (end 128.096 112.063) (width 0.2) (layer "F.Cu") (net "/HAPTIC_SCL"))
 (via (at 128.096 112.063) (size 0.6) (drill 0.3) (layers "F.Cu" "B.Cu") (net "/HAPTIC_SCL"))
 (via (at 127.136112 115.088635) (size 0.6) (drill 0.3) (layers "F.Cu" "B.Cu") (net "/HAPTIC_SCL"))
 (segment (start 127.136112 115.088635) (end 127.136112 113.022888) (width 0.2) (layer "B.Cu") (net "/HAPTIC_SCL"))
 (segment (start 127.136112 113.022888) (end 128.096 112.063) (width 0.2) (layer "B.Cu") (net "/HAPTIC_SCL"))
 (segment (start 126.251 115.035) (end 126.351 114.935) (width 0.2) (layer "F.Cu") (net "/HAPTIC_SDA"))
 (segment (start 127.471 111.238) (end 128.121 110.588) (width 0.2) (layer "F.Cu") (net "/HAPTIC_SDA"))
 (segment (start 126.251 118.95) (end 126.251 115.035) (width 0.2) (layer "F.Cu") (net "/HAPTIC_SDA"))
 (segment (start 126.446 111.238) (end 127.471 111.238) (width 0.2) (layer "F.Cu") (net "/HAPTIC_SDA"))
 (via (at 128.121 110.588) (size 0.6) (drill 0.3) (layers "F.Cu" "B.Cu") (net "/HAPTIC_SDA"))
 (via (at 126.351 114.935) (size 0.6) (drill 0.3) (layers "F.Cu" "B.Cu") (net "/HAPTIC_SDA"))
 (segment (start 126.351 112.358) (end 128.121 110.588) (width 0.2) (layer "B.Cu") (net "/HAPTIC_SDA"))
 (segment (start 126.351 114.935) (end 126.351 112.358) (width 0.2) (layer "B.Cu") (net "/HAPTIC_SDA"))
 (segment (start 128.821 112.575648) (end 129.413 113.167648) (width 0.2) (layer "F.Cu") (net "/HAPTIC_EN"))
 (segment (start 128.533648 109.813) (end 128.821 110.100352) (width 0.2) (layer "F.Cu") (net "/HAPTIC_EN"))
 (segment (start 129.413 115.988) (end 127.251 118.15) (width 0.2) (layer "F.Cu") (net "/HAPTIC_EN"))
 (segment (start 127.251 118.15) (end 127.251 118.95) (width 0.2) (layer "F.Cu") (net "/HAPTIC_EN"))
 (segment (start 126.871 109.813) (end 128.533648 109.813) (width 0.2) (layer "F.Cu") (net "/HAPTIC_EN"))
 (segment (start 126.446 110.238) (end 126.871 109.813) (width 0.2) (layer "F.Cu") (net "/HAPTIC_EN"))
 (segment (start 128.821 110.100352) (end 128.821 112.575648) (width 0.2) (layer "F.Cu") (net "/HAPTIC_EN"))
 (segment (start 129.413 113.167648) (end 129.413 115.988) (width 0.2) (layer "F.Cu") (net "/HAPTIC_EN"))
 (segment (start 117.469 110.738) (end 122.146 110.738) (width 0.2) (layer "F.Cu") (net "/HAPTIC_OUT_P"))
 (segment (start 116.205 109.474) (end 117.469 110.738) (width 0.2) (layer "F.Cu") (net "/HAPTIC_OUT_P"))
 (segment (start 116.205 114.074) (end 118.541 111.738) (width 0.2) (layer "F.Cu") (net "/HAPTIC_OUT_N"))
 (segment (start 118.541 111.738) (end 122.146 111.738) (width 0.2) (layer "F.Cu") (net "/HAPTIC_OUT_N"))
 (segment (start 128.620421 117.346265) (end 128.903265 117.346265) (width 0.2) (layer "F.Cu") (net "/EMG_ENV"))
 (segment (start 127.751 118.215686) (end 128.620421 117.346265) (width 0.2) (layer "F.Cu") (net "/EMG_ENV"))
 (segment (start 127.751 118.95) (end 127.751 118.215686) (width 0.2) (layer "F.Cu") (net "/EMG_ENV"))
 (via (at 128.903265 117.346265) (size 0.6) (drill 0.3) (layers "F.Cu" "B.Cu") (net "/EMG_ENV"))
 (via (at 117.126 105.283) (size 0.6) (drill 0.3) (layers "F.Cu" "B.Cu") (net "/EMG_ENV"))
 (segment (start 128.903265 117.346265) (end 126.255736 117.346265) (width 0.2) (layer "B.Cu") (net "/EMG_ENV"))
 (segment (start 117.643235 108.733764) (end 117.643235 105.800235) (width 0.2) (layer "B.Cu") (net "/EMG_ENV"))
 (segment (start 126.255736 117.346265) (end 117.643235 108.733764) (width 0.2) (layer "B.Cu") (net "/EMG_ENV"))
 (segment (start 117.643235 105.800235) (end 117.126 105.283) (width 0.2) (layer "B.Cu") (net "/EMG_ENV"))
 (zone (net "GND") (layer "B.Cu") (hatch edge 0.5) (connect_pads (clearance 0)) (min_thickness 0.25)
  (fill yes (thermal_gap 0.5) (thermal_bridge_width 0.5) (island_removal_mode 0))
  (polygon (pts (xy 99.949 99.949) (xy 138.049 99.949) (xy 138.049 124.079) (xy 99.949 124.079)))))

